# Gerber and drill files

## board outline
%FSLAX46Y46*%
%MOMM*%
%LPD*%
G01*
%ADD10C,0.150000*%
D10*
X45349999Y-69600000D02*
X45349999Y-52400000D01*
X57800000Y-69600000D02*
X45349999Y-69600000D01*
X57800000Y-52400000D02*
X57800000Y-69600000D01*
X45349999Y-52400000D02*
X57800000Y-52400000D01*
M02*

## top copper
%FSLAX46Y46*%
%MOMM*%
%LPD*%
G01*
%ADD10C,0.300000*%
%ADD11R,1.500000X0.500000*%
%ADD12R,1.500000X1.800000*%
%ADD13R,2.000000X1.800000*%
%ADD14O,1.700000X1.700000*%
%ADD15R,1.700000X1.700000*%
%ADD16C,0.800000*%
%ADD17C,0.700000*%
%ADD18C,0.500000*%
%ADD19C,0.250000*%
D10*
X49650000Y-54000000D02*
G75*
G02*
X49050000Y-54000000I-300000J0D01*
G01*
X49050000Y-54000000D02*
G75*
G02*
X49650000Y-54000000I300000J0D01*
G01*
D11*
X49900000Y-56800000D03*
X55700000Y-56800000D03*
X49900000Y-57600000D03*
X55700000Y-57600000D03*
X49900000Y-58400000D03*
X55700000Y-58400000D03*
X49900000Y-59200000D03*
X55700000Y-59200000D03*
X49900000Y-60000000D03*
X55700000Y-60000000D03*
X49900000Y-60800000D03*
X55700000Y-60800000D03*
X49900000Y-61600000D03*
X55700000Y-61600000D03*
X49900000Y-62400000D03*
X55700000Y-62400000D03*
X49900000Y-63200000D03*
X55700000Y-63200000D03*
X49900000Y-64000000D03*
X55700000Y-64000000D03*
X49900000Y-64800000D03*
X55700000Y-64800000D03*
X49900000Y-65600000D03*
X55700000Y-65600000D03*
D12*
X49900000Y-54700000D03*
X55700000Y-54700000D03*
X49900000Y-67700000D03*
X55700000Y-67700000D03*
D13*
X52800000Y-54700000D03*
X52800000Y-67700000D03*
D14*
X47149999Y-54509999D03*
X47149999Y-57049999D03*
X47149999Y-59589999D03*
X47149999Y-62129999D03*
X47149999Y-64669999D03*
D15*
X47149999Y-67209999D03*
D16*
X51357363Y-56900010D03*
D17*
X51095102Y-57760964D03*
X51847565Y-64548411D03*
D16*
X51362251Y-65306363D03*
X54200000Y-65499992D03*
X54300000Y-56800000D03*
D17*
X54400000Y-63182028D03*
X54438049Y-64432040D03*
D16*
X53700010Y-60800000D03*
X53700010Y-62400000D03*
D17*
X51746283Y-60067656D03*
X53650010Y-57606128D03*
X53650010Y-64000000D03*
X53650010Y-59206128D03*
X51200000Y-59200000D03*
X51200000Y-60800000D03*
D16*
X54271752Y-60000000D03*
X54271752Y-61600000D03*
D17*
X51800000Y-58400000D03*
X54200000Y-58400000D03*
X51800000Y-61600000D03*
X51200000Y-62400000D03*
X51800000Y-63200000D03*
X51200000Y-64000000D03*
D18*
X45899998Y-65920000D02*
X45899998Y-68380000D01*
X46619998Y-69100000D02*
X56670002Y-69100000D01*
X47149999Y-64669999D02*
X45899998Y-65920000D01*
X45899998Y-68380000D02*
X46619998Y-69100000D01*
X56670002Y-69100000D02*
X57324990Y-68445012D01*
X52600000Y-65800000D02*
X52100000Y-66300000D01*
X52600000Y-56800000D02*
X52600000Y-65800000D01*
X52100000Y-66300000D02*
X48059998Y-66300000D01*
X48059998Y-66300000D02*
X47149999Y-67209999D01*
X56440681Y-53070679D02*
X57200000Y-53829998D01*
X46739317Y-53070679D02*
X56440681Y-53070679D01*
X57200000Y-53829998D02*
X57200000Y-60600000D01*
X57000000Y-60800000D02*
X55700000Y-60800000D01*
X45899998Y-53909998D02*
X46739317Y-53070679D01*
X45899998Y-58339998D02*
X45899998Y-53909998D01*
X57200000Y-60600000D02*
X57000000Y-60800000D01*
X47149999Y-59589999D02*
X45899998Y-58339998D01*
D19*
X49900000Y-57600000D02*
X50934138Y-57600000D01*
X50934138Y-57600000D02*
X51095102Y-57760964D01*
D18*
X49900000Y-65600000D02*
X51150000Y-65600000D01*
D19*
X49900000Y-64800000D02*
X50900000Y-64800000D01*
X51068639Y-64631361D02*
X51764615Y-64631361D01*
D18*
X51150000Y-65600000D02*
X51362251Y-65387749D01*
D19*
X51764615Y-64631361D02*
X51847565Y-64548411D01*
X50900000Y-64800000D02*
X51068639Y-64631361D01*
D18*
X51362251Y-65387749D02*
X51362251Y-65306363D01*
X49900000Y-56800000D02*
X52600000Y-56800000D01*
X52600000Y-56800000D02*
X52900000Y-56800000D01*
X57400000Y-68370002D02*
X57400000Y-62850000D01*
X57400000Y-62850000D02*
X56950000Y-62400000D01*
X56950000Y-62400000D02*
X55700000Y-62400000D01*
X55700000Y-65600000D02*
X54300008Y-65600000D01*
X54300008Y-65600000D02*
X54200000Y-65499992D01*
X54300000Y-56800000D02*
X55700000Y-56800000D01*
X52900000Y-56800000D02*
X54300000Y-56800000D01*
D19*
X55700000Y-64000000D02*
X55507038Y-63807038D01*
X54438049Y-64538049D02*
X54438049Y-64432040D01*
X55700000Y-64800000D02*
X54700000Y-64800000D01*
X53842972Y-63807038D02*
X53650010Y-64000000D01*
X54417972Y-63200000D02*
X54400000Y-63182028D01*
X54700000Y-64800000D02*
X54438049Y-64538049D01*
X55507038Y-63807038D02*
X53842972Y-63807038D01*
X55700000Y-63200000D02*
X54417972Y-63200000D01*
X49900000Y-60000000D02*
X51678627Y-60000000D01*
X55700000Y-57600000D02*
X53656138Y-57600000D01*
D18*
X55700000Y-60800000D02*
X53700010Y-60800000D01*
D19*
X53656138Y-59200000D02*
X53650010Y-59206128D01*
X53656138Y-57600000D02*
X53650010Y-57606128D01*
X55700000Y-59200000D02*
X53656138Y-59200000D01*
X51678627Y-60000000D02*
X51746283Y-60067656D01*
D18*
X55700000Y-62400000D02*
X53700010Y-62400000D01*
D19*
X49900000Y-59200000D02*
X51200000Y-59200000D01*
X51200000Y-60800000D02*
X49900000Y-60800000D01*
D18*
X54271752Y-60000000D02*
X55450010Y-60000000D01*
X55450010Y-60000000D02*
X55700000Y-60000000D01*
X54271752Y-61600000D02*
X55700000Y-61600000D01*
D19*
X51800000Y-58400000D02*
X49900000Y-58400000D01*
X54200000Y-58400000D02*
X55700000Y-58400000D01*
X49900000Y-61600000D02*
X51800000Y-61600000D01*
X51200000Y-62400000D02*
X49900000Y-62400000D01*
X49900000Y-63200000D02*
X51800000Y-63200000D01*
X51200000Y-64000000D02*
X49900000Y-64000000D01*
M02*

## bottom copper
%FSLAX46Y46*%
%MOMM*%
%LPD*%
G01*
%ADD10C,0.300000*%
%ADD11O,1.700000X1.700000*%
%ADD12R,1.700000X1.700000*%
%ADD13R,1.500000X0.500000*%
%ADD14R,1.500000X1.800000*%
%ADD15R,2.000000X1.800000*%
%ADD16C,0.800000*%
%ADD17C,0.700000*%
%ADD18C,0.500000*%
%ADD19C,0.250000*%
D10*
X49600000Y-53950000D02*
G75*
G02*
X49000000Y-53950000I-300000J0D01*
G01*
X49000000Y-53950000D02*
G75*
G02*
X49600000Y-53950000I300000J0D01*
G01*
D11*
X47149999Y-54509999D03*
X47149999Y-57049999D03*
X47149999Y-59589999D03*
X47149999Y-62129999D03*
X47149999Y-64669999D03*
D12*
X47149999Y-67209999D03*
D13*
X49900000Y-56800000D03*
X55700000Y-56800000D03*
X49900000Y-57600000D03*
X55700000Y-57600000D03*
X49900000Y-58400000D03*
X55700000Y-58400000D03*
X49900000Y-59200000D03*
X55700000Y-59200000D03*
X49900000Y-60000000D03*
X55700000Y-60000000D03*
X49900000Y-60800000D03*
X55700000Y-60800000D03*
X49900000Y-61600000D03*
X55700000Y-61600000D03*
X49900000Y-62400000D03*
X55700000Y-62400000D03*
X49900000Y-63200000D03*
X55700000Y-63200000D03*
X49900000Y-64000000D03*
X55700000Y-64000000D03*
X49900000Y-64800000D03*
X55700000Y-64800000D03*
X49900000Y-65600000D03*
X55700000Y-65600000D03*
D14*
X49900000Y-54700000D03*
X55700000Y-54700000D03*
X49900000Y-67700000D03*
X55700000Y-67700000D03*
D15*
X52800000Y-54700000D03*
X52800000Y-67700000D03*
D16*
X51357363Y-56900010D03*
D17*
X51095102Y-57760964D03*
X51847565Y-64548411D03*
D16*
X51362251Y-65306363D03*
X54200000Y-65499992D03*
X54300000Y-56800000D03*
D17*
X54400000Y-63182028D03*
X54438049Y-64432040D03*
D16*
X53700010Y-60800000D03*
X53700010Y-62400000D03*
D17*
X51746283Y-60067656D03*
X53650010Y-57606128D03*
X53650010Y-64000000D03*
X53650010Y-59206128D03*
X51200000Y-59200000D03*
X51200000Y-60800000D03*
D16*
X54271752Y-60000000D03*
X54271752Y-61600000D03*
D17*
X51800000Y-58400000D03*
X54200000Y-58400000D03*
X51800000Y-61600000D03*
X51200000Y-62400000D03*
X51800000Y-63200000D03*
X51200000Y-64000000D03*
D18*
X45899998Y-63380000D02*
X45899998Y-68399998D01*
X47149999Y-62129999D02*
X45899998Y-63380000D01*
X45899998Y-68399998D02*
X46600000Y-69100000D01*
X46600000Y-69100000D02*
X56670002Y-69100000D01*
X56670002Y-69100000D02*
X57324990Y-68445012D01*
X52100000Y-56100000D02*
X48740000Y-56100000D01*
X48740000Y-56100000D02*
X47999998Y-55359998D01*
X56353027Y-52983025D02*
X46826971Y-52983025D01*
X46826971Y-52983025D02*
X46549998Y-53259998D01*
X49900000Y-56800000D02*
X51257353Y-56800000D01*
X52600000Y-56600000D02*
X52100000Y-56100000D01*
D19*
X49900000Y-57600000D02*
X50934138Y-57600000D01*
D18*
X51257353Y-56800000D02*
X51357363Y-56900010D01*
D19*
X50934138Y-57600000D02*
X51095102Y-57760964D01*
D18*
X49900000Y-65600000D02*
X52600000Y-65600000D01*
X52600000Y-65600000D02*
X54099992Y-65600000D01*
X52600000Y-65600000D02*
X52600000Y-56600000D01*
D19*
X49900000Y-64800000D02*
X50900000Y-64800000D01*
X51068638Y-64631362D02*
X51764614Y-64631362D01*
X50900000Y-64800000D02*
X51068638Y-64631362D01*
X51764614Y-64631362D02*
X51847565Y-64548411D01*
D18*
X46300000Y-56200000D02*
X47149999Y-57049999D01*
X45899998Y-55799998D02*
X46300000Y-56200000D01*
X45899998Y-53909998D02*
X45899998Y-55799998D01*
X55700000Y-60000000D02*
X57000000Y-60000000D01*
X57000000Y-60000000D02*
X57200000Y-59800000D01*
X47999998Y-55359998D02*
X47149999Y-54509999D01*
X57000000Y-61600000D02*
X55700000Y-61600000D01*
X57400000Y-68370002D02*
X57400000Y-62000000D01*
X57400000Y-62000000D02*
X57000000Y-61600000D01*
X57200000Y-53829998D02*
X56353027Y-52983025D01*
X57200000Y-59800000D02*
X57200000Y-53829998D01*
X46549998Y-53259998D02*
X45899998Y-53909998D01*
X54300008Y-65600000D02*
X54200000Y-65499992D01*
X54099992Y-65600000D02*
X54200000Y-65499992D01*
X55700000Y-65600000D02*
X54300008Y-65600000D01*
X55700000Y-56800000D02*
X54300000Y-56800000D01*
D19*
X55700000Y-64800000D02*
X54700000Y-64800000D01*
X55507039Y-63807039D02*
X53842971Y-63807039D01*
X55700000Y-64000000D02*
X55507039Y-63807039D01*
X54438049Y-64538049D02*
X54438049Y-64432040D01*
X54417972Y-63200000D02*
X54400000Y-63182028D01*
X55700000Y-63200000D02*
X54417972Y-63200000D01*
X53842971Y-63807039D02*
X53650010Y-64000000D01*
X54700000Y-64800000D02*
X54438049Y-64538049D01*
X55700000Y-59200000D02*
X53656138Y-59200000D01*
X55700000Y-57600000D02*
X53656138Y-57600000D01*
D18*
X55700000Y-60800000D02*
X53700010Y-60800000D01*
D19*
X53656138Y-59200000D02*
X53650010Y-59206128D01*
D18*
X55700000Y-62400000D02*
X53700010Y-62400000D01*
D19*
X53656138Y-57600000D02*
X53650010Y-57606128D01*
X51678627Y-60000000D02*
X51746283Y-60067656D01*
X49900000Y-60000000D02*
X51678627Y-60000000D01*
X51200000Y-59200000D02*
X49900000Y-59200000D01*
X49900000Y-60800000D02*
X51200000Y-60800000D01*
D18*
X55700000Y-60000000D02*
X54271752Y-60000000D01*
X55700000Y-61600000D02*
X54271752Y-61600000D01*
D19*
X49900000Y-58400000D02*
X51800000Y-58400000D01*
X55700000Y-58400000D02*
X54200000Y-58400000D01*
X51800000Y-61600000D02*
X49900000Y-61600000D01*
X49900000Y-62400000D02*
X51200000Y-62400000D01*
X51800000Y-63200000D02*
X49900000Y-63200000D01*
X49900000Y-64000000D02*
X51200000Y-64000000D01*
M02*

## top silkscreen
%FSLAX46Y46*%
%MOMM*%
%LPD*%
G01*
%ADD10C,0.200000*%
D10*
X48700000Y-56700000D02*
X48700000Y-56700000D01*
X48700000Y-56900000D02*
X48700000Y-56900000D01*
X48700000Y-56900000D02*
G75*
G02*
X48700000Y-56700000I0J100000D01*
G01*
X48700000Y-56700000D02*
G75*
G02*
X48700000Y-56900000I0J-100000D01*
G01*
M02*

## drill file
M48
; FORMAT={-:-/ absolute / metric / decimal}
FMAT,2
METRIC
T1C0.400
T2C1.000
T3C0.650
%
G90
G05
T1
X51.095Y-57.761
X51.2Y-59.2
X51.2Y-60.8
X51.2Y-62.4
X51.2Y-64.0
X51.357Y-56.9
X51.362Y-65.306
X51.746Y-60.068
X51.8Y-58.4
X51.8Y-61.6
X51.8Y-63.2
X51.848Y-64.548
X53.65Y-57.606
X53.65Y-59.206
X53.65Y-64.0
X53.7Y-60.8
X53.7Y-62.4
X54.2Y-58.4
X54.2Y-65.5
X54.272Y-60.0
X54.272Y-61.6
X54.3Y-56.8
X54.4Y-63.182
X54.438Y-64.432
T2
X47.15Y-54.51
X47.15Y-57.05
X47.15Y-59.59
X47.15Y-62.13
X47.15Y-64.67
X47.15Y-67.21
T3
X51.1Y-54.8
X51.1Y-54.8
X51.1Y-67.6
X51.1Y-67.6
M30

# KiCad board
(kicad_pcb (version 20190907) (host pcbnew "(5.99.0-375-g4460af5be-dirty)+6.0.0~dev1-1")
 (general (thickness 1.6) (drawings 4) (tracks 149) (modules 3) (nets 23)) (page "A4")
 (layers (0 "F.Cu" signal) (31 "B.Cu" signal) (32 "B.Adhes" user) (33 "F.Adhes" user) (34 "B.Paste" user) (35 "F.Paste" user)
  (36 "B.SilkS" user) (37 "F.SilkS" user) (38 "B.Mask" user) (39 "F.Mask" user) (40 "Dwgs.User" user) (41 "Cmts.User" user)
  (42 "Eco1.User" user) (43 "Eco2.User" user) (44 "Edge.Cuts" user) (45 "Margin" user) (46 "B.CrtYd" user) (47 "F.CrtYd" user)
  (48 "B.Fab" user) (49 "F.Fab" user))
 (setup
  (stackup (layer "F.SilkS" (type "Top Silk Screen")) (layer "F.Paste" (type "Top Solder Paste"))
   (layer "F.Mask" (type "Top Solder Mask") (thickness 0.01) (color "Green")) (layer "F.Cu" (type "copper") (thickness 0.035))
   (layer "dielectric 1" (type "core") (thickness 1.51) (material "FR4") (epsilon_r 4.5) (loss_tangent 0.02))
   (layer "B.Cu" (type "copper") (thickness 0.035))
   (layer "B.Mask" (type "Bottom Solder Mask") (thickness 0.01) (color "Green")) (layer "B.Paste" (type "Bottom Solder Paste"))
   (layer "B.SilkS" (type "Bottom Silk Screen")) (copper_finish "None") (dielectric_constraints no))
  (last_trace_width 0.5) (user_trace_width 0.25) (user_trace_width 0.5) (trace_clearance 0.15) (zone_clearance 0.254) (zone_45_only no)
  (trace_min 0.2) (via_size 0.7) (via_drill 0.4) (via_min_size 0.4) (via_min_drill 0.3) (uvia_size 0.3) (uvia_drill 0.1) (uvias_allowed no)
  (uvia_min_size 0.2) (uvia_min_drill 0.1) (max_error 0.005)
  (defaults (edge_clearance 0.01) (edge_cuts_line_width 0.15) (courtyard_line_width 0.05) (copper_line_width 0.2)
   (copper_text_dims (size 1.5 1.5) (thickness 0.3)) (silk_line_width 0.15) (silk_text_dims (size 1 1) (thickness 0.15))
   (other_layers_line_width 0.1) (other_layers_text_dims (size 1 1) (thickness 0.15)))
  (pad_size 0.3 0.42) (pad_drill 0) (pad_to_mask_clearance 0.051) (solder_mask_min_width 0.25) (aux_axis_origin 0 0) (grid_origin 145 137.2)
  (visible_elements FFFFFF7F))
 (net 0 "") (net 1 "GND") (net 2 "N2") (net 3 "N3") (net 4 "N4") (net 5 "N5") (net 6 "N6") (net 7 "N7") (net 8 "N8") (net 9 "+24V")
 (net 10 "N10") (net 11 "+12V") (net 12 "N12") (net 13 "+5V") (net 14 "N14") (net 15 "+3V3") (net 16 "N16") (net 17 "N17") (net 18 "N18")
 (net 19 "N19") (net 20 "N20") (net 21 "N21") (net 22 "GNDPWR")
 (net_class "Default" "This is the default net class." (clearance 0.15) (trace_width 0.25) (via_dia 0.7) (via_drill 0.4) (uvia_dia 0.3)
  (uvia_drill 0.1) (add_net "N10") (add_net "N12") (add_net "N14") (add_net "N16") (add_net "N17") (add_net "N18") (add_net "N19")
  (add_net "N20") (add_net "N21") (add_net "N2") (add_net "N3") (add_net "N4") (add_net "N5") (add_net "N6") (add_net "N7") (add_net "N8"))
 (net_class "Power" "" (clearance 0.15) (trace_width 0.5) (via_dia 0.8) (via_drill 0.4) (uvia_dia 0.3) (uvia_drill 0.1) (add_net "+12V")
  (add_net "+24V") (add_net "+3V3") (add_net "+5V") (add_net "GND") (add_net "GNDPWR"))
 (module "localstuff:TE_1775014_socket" (layer "F.Cu") (at 52.8 61.2 -90)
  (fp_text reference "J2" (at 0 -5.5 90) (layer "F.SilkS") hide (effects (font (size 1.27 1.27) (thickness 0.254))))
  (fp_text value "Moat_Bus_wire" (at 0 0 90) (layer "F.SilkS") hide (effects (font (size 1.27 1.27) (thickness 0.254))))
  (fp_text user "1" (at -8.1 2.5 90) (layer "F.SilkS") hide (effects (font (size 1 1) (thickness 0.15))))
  (fp_circle (center -7.2 3.45) (end -6.9 3.45) (layer "F.Cu") (width 0.3))
  (fp_line (start -4.5 4.1) (end -4.5 4.1) (layer "F.SilkS") (width 0.2))
  (fp_line (start -4.3 4.1) (end -4.3 4.1) (layer "F.SilkS") (width 0.2))
  (fp_arc (start -4.4 4.1) (end -4.5 4.1) (angle -180) (layer "F.SilkS") (width 0.2))
  (fp_arc (start -4.4 4.1) (end -4.3 4.1) (angle -180) (layer "F.SilkS") (width 0.2))
  (pad "1" smd rect (at -4.4 2.9 270) (size 0.5 1.5) (layers "F.Cu" "F.Paste" "F.Mask") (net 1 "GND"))
  (pad "2" smd rect (at -4.4 -2.9 270) (size 0.5 1.5) (layers "F.Cu" "F.Paste" "F.Mask") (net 1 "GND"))
  (pad "3" smd rect (at -3.6 2.9 270) (size 0.5 1.5) (layers "F.Cu" "F.Paste" "F.Mask") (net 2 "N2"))
  (pad "4" smd rect (at -3.6 -2.9 270) (size 0.5 1.5) (layers "F.Cu" "F.Paste" "F.Mask") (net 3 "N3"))
  (pad "5" smd rect (at -2.8 2.9 270) (size 0.5 1.5) (layers "F.Cu" "F.Paste" "F.Mask") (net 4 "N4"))
  (pad "6" smd rect (at -2.8 -2.9 270) (size 0.5 1.5) (layers "F.Cu" "F.Paste" "F.Mask") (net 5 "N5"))
  (pad "7" smd rect (at -2 2.9 270) (size 0.5 1.5) (layers "F.Cu" "F.Paste" "F.Mask") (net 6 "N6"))
  (pad "8" smd rect (at -2 -2.9 270) (size 0.5 1.5) (layers "F.Cu" "F.Paste" "F.Mask") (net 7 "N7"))
  (pad "9" smd rect (at -1.2 2.9 270) (size 0.5 1.5) (layers "F.Cu" "F.Paste" "F.Mask") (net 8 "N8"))
  (pad "10" smd rect (at -1.2 -2.9 270) (size 0.5 1.5) (layers "F.Cu" "F.Paste" "F.Mask") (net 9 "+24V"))
  (pad "11" smd rect (at -0.4 2.9 270) (size 0.5 1.5) (layers "F.Cu" "F.Paste" "F.Mask") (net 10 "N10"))
  (pad "12" smd rect (at -0.4 -2.9 270) (size 0.5 1.5) (layers "F.Cu" "F.Paste" "F.Mask") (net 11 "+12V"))
  (pad "13" smd rect (at 0.4 2.9 270) (size 0.5 1.5) (layers "F.Cu" "F.Paste" "F.Mask") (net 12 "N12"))
  (pad "14" smd rect (at 0.4 -2.9 270) (size 0.5 1.5) (layers "F.Cu" "F.Paste" "F.Mask") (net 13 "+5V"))
  (pad "15" smd rect (at 1.2 2.9 270) (size 0.5 1.5) (layers "F.Cu" "F.Paste" "F.Mask") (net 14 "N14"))
  (pad "16" smd rect (at 1.2 -2.9 270) (size 0.5 1.5) (layers "F.Cu" "F.Paste" "F.Mask") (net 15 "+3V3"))
  (pad "17" smd rect (at 2 2.9 270) (size 0.5 1.5) (layers "F.Cu" "F.Paste" "F.Mask") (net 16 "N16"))
  (pad "18" smd rect (at 2 -2.9 270) (size 0.5 1.5) (layers "F.Cu" "F.Paste" "F.Mask") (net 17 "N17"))
  (pad "19" smd rect (at 2.8 2.9 270) (size 0.5 1.5) (layers "F.Cu" "F.Paste" "F.Mask") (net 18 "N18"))
  (pad "20" smd rect (at 2.8 -2.9 270) (size 0.5 1.5) (layers "F.Cu" "F.Paste" "F.Mask") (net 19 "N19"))
  (pad "21" smd rect (at 3.6 2.9 270) (size 0.5 1.5) (layers "F.Cu" "F.Paste" "F.Mask") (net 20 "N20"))
  (pad "22" smd rect (at 3.6 -2.9 270) (size 0.5 1.5) (layers "F.Cu" "F.Paste" "F.Mask") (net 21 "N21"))
  (pad "23" smd rect (at 4.4 2.9 270) (size 0.5 1.5) (layers "F.Cu" "F.Paste" "F.Mask") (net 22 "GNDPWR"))
  (pad "24" smd rect (at 4.4 -2.9 270) (size 0.5 1.5) (layers "F.Cu" "F.Paste" "F.Mask") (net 22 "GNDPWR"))
  (pad "MNT" smd rect (at -6.5 2.9) (size 1.5 1.8) (layers "F.Cu" "F.Paste" "F.Mask") (solder_paste_margin -0.05) (clearance 0.001))
  (pad "MNT" smd rect (at -6.5 -2.9) (size 1.5 1.8) (layers "F.Cu" "F.Paste" "F.Mask"))
  (pad "MNT" smd rect (at 6.5 2.9) (size 1.5 1.8) (layers "F.Cu" "F.Paste" "F.Mask") (solder_paste_margin -0.05) (clearance 0.001))
  (pad "MNT" smd rect (at 6.5 -2.9) (size 1.5 1.8) (layers "F.Cu" "F.Paste" "F.Mask"))
  (pad "MNT" smd rect (at -6.5 0 270) (size 1.8 2) (layers "F.Cu" "F.Paste" "F.Mask"))
  (pad "MNT" smd rect (at 6.5 0 270) (size 1.8 2) (layers "F.Cu" "F.Paste" "F.Mask"))
  (pad "" np_thru_hole circle (at -6.4 1.7 270) (size 0.65 0.65) (drill 0.65) (layers *.Cu *.Mask) (clearance 0.01))
  (pad "" np_thru_hole circle (at 6.4 1.7 270) (size 0.65 0.65) (drill 0.65) (layers *.Cu *.Mask) (clearance 0.0001)))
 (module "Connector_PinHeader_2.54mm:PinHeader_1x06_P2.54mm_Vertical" (layer "B.Cu") (at 47.149999 67.209999)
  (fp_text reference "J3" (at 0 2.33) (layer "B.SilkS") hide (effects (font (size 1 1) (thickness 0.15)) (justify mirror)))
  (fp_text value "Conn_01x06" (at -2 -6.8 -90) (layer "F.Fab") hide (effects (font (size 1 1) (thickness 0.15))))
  (pad "6" thru_hole oval (at 0 -12.7) (size 1.7 1.7) (drill 1) (layers *.Cu *.Mask) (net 22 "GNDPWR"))
  (pad "5" thru_hole oval (at 0 -10.16) (size 1.7 1.7) (drill 1) (layers *.Cu *.Mask) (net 9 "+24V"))
  (pad "4" thru_hole oval (at 0 -7.62) (size 1.7 1.7) (drill 1) (layers *.Cu *.Mask) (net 11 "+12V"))
  (pad "3" thru_hole oval (at 0 -5.08) (size 1.7 1.7) (drill 1) (layers *.Cu *.Mask) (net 13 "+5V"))
  (pad "2" thru_hole oval (at 0 -2.54) (size 1.7 1.7) (drill 1) (layers *.Cu *.Mask) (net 15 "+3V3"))
  (pad "1" thru_hole rect (at 0 0) (size 1.7 1.7) (drill 1) (layers *.Cu *.Mask) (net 1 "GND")))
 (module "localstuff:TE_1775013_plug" (layer "B.Cu") (at 52.8 61.2 90)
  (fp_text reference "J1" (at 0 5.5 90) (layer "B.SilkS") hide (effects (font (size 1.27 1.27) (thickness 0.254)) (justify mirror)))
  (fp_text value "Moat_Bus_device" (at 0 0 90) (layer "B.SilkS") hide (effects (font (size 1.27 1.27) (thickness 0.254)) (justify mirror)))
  (fp_circle (center 7.25 -3.5) (end 7.55 -3.5) (layer "B.Cu") (width 0.3))
  (pad "1" smd rect (at 4.4 -2.9 90) (size 0.5 1.5) (layers "B.Cu" "B.Paste" "B.Mask") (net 1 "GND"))
  (pad "2" smd rect (at 4.4 2.9 90) (size 0.5 1.5) (layers "B.Cu" "B.Paste" "B.Mask") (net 1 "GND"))
  (pad "3" smd rect (at 3.6 -2.9 90) (size 0.5 1.5) (layers "B.Cu" "B.Paste" "B.Mask") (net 2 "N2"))
  (pad "4" smd rect (at 3.6 2.9 90) (size 0.5 1.5) (layers "B.Cu" "B.Paste" "B.Mask") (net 3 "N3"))
  (pad "5" smd rect (at 2.8 -2.9 90) (size 0.5 1.5) (layers "B.Cu" "B.Paste" "B.Mask") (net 4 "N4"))
  (pad "6" smd rect (at 2.8 2.9 90) (size 0.5 1.5) (layers "B.Cu" "B.Paste" "B.Mask") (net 5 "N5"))
  (pad "7" smd rect (at 2 -2.9 90) (size 0.5 1.5) (layers "B.Cu" "B.Paste" "B.Mask") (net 6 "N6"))
  (pad "8" smd rect (at 2 2.9 90) (size 0.5 1.5) (layers "B.Cu" "B.Paste" "B.Mask") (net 7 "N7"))
  (pad "9" smd rect (at 1.2 -2.9 90) (size 0.5 1.5) (layers "B.Cu" "B.Paste" "B.Mask") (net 8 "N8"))
  (pad "10" smd rect (at 1.2 2.9 90) (size 0.5 1.5) (layers "B.Cu" "B.Paste" "B.Mask") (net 9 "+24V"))
  (pad "11" smd rect (at 0.4 -2.9 90) (size 0.5 1.5) (layers "B.Cu" "B.Paste" "B.Mask") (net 10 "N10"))
  (pad "12" smd rect (at 0.4 2.9 90) (size 0.5 1.5) (layers "B.Cu" "B.Paste" "B.Mask") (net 11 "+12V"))
  (pad "13" smd rect (at -0.4 -2.9 90) (size 0.5 1.5) (layers "B.Cu" "B.Paste" "B.Mask") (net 12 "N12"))
  (pad "14" smd rect (at -0.4 2.9 90) (size 0.5 1.5) (layers "B.Cu" "B.Paste" "B.Mask") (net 13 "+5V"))
  (pad "15" smd rect (at -1.2 -2.9 90) (size 0.5 1.5) (layers "B.Cu" "B.Paste" "B.Mask") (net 14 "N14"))
  (pad "16" smd rect (at -1.2 2.9 90) (size 0.5 1.5) (layers "B.Cu" "B.Paste" "B.Mask") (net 15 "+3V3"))
  (pad "17" smd rect (at -2 -2.9 90) (size 0.5 1.5) (layers "B.Cu" "B.Paste" "B.Mask") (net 16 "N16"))
  (pad "18" smd rect (at -2 2.9 90) (size 0.5 1.5) (layers "B.Cu" "B.Paste" "B.Mask") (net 17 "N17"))
  (pad "19" smd rect (at -2.8 -2.9 90) (size 0.5 1.5) (layers "B.Cu" "B.Paste" "B.Mask") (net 18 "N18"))
  (pad "20" smd rect (at -2.8 2.9 90) (size 0.5 1.5) (layers "B.Cu" "B.Paste" "B.Mask") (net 19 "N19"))
  (pad "21" smd rect (at -3.6 -2.9 90) (size 0.5 1.5) (layers "B.Cu" "B.Paste" "B.Mask") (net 20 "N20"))
  (pad "22" smd rect (at -3.6 2.9 90) (size 0.5 1.5) (layers "B.Cu" "B.Paste" "B.Mask") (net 21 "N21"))
  (pad "23" smd rect (at -4.4 -2.9 90) (size 0.5 1.5) (layers "B.Cu" "B.Paste" "B.Mask") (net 22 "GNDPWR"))
  (pad "24" smd rect (at -4.4 2.9 90) (size 0.5 1.5) (layers "B.Cu" "B.Paste" "B.Mask") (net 22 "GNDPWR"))
  (pad "MNT" smd rect (at 6.5 -2.9 180) (size 1.5 1.8) (layers "B.Cu" "B.Paste" "B.Mask"))
  (pad "MNT" smd rect (at 6.5 2.9 180) (size 1.5 1.8) (layers "B.Cu" "B.Paste" "B.Mask"))
  (pad "MNT" smd rect (at -6.5 -2.9 180) (size 1.5 1.8) (layers "B.Cu" "B.Paste" "B.Mask"))
  (pad "MNT" smd rect (at -6.5 2.9 180) (size 1.5 1.8) (layers "B.Cu" "B.Paste" "B.Mask"))
  (pad "MNT" smd rect (at 6.5 0 90) (size 1.8 2) (layers "B.Cu" "B.Paste" "B.Mask"))
  (pad "MNT" smd rect (at -6.5 0 90) (size 1.8 2) (layers "B.Cu" "B.Paste" "B.Mask"))
  (pad "" np_thru_hole circle (at 6.4 -1.7 90) (size 0.65 0.65) (drill 0.65) (layers *.Cu *.Mask))
  (pad "" np_thru_hole circle (at -6.4 -1.7 90) (size 0.65 0.65) (drill 0.65) (layers *.Cu *.Mask)))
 (gr_line (start 45.349999 69.6) (end 45.349999 52.4) (layer "Edge.Cuts") (width 0.15))
 (gr_line (start 57.8 69.6) (end 45.349999 69.6) (layer "Edge.Cuts") (width 0.15))
 (gr_line (start 57.8 52.4) (end 57.8 69.6) (layer "Edge.Cuts") (width 0.15))
 (gr_line (start 45.349999 52.4) (end 57.8 52.4) (layer "Edge.Cuts") (width 0.15))
 (segment (start 45.899998 63.38) (end 45.899998 68.399998) (width 0.5) (layer "B.Cu") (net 13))
 (segment (start 47.149999 62.129999) (end 45.899998 63.38) (width 0.5) (layer "B.Cu") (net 13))
 (segment (start 45.899998 68.399998) (end 46.6 69.1) (width 0.5) (layer "B.Cu") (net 13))
 (segment (start 46.6 69.1) (end 56.670002 69.1) (width 0.5) (layer "B.Cu") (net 13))
 (segment (start 56.670002 69.1) (end 57.32499 68.445012) (width 0.5) (layer "B.Cu") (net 13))
 (segment (start 45.899998 65.92) (end 45.899998 68.38) (width 0.5) (layer "F.Cu") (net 15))
 (segment (start 46.619998 69.1) (end 56.670002 69.1) (width 0.5) (layer "F.Cu") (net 15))
 (segment (start 47.149999 64.669999) (end 45.899998 65.92) (width 0.5) (layer "F.Cu") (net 15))
 (segment (start 45.899998 68.38) (end 46.619998 69.1) (width 0.5) (layer "F.Cu") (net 15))
 (segment (start 56.670002 69.1) (end 57.32499 68.445012) (width 0.5) (layer "F.Cu") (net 15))
 (segment (start 52.6 65.8) (end 52.1 66.3) (width 0.5) (layer "F.Cu") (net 1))
 (segment (start 52.6 56.8) (end 52.6 65.8) (width 0.5) (layer "F.Cu") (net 1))
 (segment (start 52.1 66.3) (end 48.059998 66.3) (width 0.5) (layer "F.Cu") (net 1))
 (segment (start 48.059998 66.3) (end 47.149999 67.209999) (width 0.5) (layer "F.Cu") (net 1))
 (segment (start 52.1 56.1) (end 48.74 56.1) (width 0.5) (layer "B.Cu") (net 22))
 (segment (start 48.74 56.1) (end 47.999998 55.359998) (width 0.5) (layer "B.Cu") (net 22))
 (segment (start 56.353027 52.983025) (end 46.826971 52.983025) (width 0.5) (layer "B.Cu") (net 9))
 (segment (start 46.826971 52.983025) (end 46.549998 53.259998) (width 0.5) (layer "B.Cu") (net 9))
 (segment (start 56.440681 53.070679) (end 57.2 53.829998) (width 0.5) (layer "F.Cu") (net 11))
 (segment (start 46.739317 53.070679) (end 56.440681 53.070679) (width 0.5) (layer "F.Cu") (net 11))
 (segment (start 57.2 53.829998) (end 57.2 60.6) (width 0.5) (layer "F.Cu") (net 11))
 (segment (start 57 60.8) (end 55.7 60.8) (width 0.5) (layer "F.Cu") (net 11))
 (segment (start 45.899998 53.909998) (end 46.739317 53.070679) (width 0.5) (layer "F.Cu") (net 11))
 (segment (start 45.899998 58.339998) (end 45.899998 53.909998) (width 0.5) (layer "F.Cu") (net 11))
 (segment (start 57.2 60.6) (end 57 60.8) (width 0.5) (layer "F.Cu") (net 11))
 (segment (start 47.149999 59.589999) (end 45.899998 58.339998) (width 0.5) (layer "F.Cu") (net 11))
 (segment (start 49.9 57.6) (end 50.934138 57.6) (width 0.25) (layer "F.Cu") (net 2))
 (segment (start 50.934138 57.6) (end 51.095102 57.760964) (width 0.25) (layer "F.Cu") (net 2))
 (segment (start 49.9 56.8) (end 51.257353 56.8) (width 0.5) (layer "B.Cu") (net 1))
 (via (at 51.357363 56.90001) (size 0.8) (drill 0.4) (layers "F.Cu" "B.Cu") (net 1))
 (segment (start 52.6 56.6) (end 52.1 56.1) (width 0.5) (layer "B.Cu") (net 22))
 (via (at 51.095102 57.760964) (size 0.7) (drill 0.4) (layers "F.Cu" "B.Cu") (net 2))
 (segment (start 49.9 57.6) (end 50.934138 57.6) (width 0.25) (layer "B.Cu") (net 2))
 (segment (start 51.257353 56.8) (end 51.357363 56.90001) (width 0.5) (layer "B.Cu") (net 1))
 (segment (start 50.934138 57.6) (end 51.095102 57.760964) (width 0.25) (layer "B.Cu") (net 2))
 (segment (start 49.9 65.6) (end 52.6 65.6) (width 0.5) (layer "B.Cu") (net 22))
 (segment (start 52.6 65.6) (end 54.099992 65.6) (width 0.5) (layer "B.Cu") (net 22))
 (segment (start 52.6 65.6) (end 52.6 56.6) (width 0.5) (layer "B.Cu") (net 22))
 (segment (start 49.9 64.8) (end 50.9 64.8) (width 0.25) (layer "B.Cu") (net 20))
 (via (at 51.847565 64.548411) (size 0.7) (drill 0.4) (layers "F.Cu" "B.Cu") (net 20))
 (segment (start 49.9 65.6) (end 51.15 65.6) (width 0.5) (layer "F.Cu") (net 22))
 (segment (start 51.068638 64.631362) (end 51.764614 64.631362) (width 0.25) (layer "B.Cu") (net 20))
 (segment (start 49.9 64.8) (end 50.9 64.8) (width 0.25) (layer "F.Cu") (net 20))
 (segment (start 51.068639 64.631361) (end 51.764615 64.631361) (width 0.25) (layer "F.Cu") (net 20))
 (segment (start 50.9 64.8) (end 51.068638 64.631362) (width 0.25) (layer "B.Cu") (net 20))
 (segment (start 51.764614 64.631362) (end 51.847565 64.548411) (width 0.25) (layer "B.Cu") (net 20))
 (segment (start 51.15 65.6) (end 51.362251 65.387749) (width 0.5) (layer "F.Cu") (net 22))
 (segment (start 51.764615 64.631361) (end 51.847565 64.548411) (width 0.25) (layer "F.Cu") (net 20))
 (via (at 51.362251 65.306363) (size 0.8) (drill 0.4) (layers "F.Cu" "B.Cu") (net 22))
 (segment (start 50.9 64.8) (end 51.068639 64.631361) (width 0.25) (layer "F.Cu") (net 20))
 (segment (start 51.362251 65.387749) (end 51.362251 65.306363) (width 0.5) (layer "F.Cu") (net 22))
 (segment (start 49.9 56.8) (end 52.6 56.8) (width 0.5) (layer "F.Cu") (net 1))
 (segment (start 52.6 56.8) (end 52.9 56.8) (width 0.5) (layer "F.Cu") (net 1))
 (segment (start 46.3 56.2) (end 47.149999 57.049999) (width 0.5) (layer "B.Cu") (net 9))
 (segment (start 45.899998 55.799998) (end 46.3 56.2) (width 0.5) (layer "B.Cu") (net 9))
 (segment (start 45.899998 53.909998) (end 45.899998 55.799998) (width 0.5) (layer "B.Cu") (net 9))
 (segment (start 55.7 60) (end 57 60) (width 0.5) (layer "B.Cu") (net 9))
 (segment (start 57 60) (end 57.2 59.8) (width 0.5) (layer "B.Cu") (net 9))
 (segment (start 47.999998 55.359998) (end 47.149999 54.509999) (width 0.5) (layer "B.Cu") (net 22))
 (segment (start 57 61.6) (end 55.7 61.6) (width 0.5) (layer "B.Cu") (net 13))
 (segment (start 57.4 68.370002) (end 57.4 62) (width 0.5) (layer "B.Cu") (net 13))
 (segment (start 57.4 62) (end 57 61.6) (width 0.5) (layer "B.Cu") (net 13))
 (segment (start 57.2 53.829998) (end 56.353027 52.983025) (width 0.5) (layer "B.Cu") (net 9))
 (segment (start 57.2 59.8) (end 57.2 53.829998) (width 0.5) (layer "B.Cu") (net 9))
 (segment (start 46.549998 53.259998) (end 45.899998 53.909998) (width 0.5) (layer "B.Cu") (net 9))
 (segment (start 57.4 68.370002) (end 57.4 62.85) (width 0.5) (layer "F.Cu") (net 15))
 (segment (start 57.4 62.85) (end 56.95 62.4) (width 0.5) (layer "F.Cu") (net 15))
 (segment (start 56.95 62.4) (end 55.7 62.4) (width 0.5) (layer "F.Cu") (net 15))
 (via (at 54.2 65.499992) (size 0.8) (drill 0.4) (layers "F.Cu" "B.Cu") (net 22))
 (segment (start 55.7 65.6) (end 54.300008 65.6) (width 0.5) (layer "F.Cu") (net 22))
 (segment (start 54.300008 65.6) (end 54.2 65.499992) (width 0.5) (layer "B.Cu") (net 22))
 (segment (start 54.099992 65.6) (end 54.2 65.499992) (width 0.5) (layer "B.Cu") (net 22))
 (segment (start 54.300008 65.6) (end 54.2 65.499992) (width 0.5) (layer "F.Cu") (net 22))
 (segment (start 55.7 65.6) (end 54.300008 65.6) (width 0.5) (layer "B.Cu") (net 22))
 (segment (start 54.3 56.8) (end 55.7 56.8) (width 0.5) (layer "F.Cu") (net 1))
 (segment (start 52.9 56.8) (end 54.3 56.8) (width 0.5) (layer "F.Cu") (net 1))
 (segment (start 55.7 56.8) (end 54.3 56.8) (width 0.5) (layer "B.Cu") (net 1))
 (via (at 54.3 56.8) (size 0.8) (drill 0.4) (layers "F.Cu" "B.Cu") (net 1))
 (segment (start 55.7 64) (end 55.507038 63.807038) (width 0.25) (layer "F.Cu") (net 19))
 (via (at 54.4 63.182028) (size 0.7) (drill 0.4) (layers "F.Cu" "B.Cu") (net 17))
 (segment (start 54.438049 64.538049) (end 54.438049 64.43204) (width 0.25) (layer "F.Cu") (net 21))
 (segment (start 55.7 64.8) (end 54.7 64.8) (width 0.25) (layer "B.Cu") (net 21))
 (segment (start 55.7 64.8) (end 54.7 64.8) (width 0.25) (layer "F.Cu") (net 21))
 (segment (start 55.507039 63.807039) (end 53.842971 63.807039) (width 0.25) (layer "B.Cu") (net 19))
 (segment (start 55.7 64) (end 55.507039 63.807039) (width 0.25) (layer "B.Cu") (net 19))
 (segment (start 53.842972 63.807038) (end 53.65001 64) (width 0.25) (layer "F.Cu") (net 19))
 (segment (start 54.438049 64.538049) (end 54.438049 64.43204) (width 0.25) (layer "B.Cu") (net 21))
 (segment (start 54.417972 63.2) (end 54.4 63.182028) (width 0.25) (layer "F.Cu") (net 17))
 (segment (start 54.417972 63.2) (end 54.4 63.182028) (width 0.25) (layer "B.Cu") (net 17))
 (segment (start 55.7 63.2) (end 54.417972 63.2) (width 0.25) (layer "B.Cu") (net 17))
 (segment (start 54.7 64.8) (end 54.438049 64.538049) (width 0.25) (layer "F.Cu") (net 21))
 (segment (start 53.842971 63.807039) (end 53.65001 64) (width 0.25) (layer "B.Cu") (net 19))
 (via (at 54.438049 64.43204) (size 0.7) (drill 0.4) (layers "F.Cu" "B.Cu") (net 21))
 (segment (start 54.7 64.8) (end 54.438049 64.538049) (width 0.25) (layer "B.Cu") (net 21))
 (segment (start 55.507038 63.807038) (end 53.842972 63.807038) (width 0.25) (layer "F.Cu") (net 19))
 (segment (start 55.7 63.2) (end 54.417972 63.2) (width 0.25) (layer "F.Cu") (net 17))
 (segment (start 49.9 60) (end 51.678627 60) (width 0.25) (layer "F.Cu") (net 8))
 (segment (start 55.7 59.2) (end 53.656138 59.2) (width 0.25) (layer "B.Cu") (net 7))
 (segment (start 55.7 57.6) (end 53.656138 57.6) (width 0.25) (layer "F.Cu") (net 3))
 (via (at 53.70001 60.8) (size 0.8) (drill 0.4) (layers "F.Cu" "B.Cu") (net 11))
 (via (at 53.70001 62.4) (size 0.8) (drill 0.4) (layers "F.Cu" "B.Cu") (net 15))
 (segment (start 55.7 57.6) (end 53.656138 57.6) (width 0.25) (layer "B.Cu") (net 3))
 (segment (start 55.7 60.8) (end 53.70001 60.8) (width 0.5) (layer "F.Cu") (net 11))
 (via (at 51.746283 60.067656) (size 0.7) (drill 0.4) (layers "F.Cu" "B.Cu") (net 8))
 (segment (start 53.656138 59.2) (end 53.65001 59.206128) (width 0.25) (layer "F.Cu") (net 7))
 (via (at 53.65001 57.606128) (size 0.7) (drill 0.4) (layers "F.Cu" "B.Cu") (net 3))
 (segment (start 53.656138 57.6) (end 53.65001 57.606128) (width 0.25) (layer "F.Cu") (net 3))
 (segment (start 55.7 60.8) (end 53.70001 60.8) (width 0.5) (layer "B.Cu") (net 11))
 (segment (start 53.656138 59.2) (end 53.65001 59.206128) (width 0.25) (layer "B.Cu") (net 7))
 (segment (start 55.7 62.4) (end 53.70001 62.4) (width 0.5) (layer "B.Cu") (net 15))
 (segment (start 53.656138 57.6) (end 53.65001 57.606128) (width 0.25) (layer "B.Cu") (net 3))
 (via (at 53.65001 64) (size 0.7) (drill 0.4) (layers "F.Cu" "B.Cu") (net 19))
 (segment (start 55.7 59.2) (end 53.656138 59.2) (width 0.25) (layer "F.Cu") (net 7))
 (segment (start 51.678627 60) (end 51.746283 60.067656) (width 0.25) (layer "F.Cu") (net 8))
 (segment (start 51.678627 60) (end 51.746283 60.067656) (width 0.25) (layer "B.Cu") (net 8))
 (segment (start 49.9 60) (end 51.678627 60) (width 0.25) (layer "B.Cu") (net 8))
 (segment (start 55.7 62.4) (end 53.70001 62.4) (width 0.5) (layer "F.Cu") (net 15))
 (via (at 53.65001 59.206128) (size 0.7) (drill 0.4) (layers "F.Cu" "B.Cu") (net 7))
 (via (at 51.2 59.2) (size 0.7) (drill 0.4) (layers "F.Cu" "B.Cu") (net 6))
 (segment (start 49.9 59.2) (end 51.2 59.2) (width 0.25) (layer "F.Cu") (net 6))
 (segment (start 51.2 59.2) (end 49.9 59.2) (width 0.25) (layer "B.Cu") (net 6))
 (via (at 51.2 60.8) (size 0.7) (drill 0.4) (layers "F.Cu" "B.Cu") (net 10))
 (segment (start 49.9 60.8) (end 51.2 60.8) (width 0.25) (layer "B.Cu") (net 10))
 (segment (start 51.2 60.8) (end 49.9 60.8) (width 0.25) (layer "F.Cu") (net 10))
 (via (at 54.271752 60) (size 0.8) (drill 0.4) (layers "F.Cu" "B.Cu") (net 9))
 (segment (start 55.7 60) (end 54.271752 60) (width 0.5) (layer "B.Cu") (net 9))
 (segment (start 54.271752 60) (end 55.45001 60) (width 0.5) (layer "F.Cu") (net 9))
 (segment (start 55.45001 60) (end 55.7 60) (width 0.5) (layer "F.Cu") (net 9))
 (via (at 54.271752 61.6) (size 0.8) (drill 0.4) (layers "F.Cu" "B.Cu") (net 13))
 (segment (start 55.7 61.6) (end 54.271752 61.6) (width 0.5) (layer "B.Cu") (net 13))
 (segment (start 54.271752 61.6) (end 55.7 61.6) (width 0.5) (layer "F.Cu") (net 13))
 (via (at 51.8 58.4) (size 0.7) (drill 0.4) (layers "F.Cu" "B.Cu") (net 4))
 (segment (start 49.9 58.4) (end 51.8 58.4) (width 0.25) (layer "B.Cu") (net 4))
 (segment (start 51.8 58.4) (end 49.9 58.4) (width 0.25) (layer "F.Cu") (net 4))
 (via (at 54.2 58.4) (size 0.7) (drill 0.4) (layers "F.Cu" "B.Cu") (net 5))
 (segment (start 55.7 58.4) (end 54.2 58.4) (width 0.25) (layer "B.Cu") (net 5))
 (segment (start 54.2 58.4) (end 55.7 58.4) (width 0.25) (layer "F.Cu") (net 5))
 (via (at 51.8 61.6) (size 0.7) (drill 0.4) (layers "F.Cu" "B.Cu") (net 12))
 (segment (start 49.9 61.6) (end 51.8 61.6) (width 0.25) (layer "F.Cu") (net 12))
 (segment (start 51.8 61.6) (end 49.9 61.6) (width 0.25) (layer "B.Cu") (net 12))
 (via (at 51.2 62.4) (size 0.7) (drill 0.4) (layers "F.Cu" "B.Cu") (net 14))
 (segment (start 49.9 62.4) (end 51.2 62.4) (width 0.25) (layer "B.Cu") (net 14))
 (segment (start 51.2 62.4) (end 49.9 62.4) (width 0.25) (layer "F.Cu") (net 14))
 (via (at 51.8 63.2) (size 0.7) (drill 0.4) (layers "F.Cu" "B.Cu") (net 16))
 (segment (start 49.9 63.2) (end 51.8 63.2) (width 0.25) (layer "F.Cu") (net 16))
 (segment (start 51.8 63.2) (end 49.9 63.2) (width 0.25) (layer "B.Cu") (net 16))
 (via (at 51.2 64) (size 0.7) (drill 0.4) (layers "F.Cu" "B.Cu") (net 18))
 (segment (start 49.9 64) (end 51.2 64) (width 0.25) (layer "B.Cu") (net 18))
 (segment (start 51.2 64) (end 49.9 64) (width 0.25) (layer "F.Cu") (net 18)))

